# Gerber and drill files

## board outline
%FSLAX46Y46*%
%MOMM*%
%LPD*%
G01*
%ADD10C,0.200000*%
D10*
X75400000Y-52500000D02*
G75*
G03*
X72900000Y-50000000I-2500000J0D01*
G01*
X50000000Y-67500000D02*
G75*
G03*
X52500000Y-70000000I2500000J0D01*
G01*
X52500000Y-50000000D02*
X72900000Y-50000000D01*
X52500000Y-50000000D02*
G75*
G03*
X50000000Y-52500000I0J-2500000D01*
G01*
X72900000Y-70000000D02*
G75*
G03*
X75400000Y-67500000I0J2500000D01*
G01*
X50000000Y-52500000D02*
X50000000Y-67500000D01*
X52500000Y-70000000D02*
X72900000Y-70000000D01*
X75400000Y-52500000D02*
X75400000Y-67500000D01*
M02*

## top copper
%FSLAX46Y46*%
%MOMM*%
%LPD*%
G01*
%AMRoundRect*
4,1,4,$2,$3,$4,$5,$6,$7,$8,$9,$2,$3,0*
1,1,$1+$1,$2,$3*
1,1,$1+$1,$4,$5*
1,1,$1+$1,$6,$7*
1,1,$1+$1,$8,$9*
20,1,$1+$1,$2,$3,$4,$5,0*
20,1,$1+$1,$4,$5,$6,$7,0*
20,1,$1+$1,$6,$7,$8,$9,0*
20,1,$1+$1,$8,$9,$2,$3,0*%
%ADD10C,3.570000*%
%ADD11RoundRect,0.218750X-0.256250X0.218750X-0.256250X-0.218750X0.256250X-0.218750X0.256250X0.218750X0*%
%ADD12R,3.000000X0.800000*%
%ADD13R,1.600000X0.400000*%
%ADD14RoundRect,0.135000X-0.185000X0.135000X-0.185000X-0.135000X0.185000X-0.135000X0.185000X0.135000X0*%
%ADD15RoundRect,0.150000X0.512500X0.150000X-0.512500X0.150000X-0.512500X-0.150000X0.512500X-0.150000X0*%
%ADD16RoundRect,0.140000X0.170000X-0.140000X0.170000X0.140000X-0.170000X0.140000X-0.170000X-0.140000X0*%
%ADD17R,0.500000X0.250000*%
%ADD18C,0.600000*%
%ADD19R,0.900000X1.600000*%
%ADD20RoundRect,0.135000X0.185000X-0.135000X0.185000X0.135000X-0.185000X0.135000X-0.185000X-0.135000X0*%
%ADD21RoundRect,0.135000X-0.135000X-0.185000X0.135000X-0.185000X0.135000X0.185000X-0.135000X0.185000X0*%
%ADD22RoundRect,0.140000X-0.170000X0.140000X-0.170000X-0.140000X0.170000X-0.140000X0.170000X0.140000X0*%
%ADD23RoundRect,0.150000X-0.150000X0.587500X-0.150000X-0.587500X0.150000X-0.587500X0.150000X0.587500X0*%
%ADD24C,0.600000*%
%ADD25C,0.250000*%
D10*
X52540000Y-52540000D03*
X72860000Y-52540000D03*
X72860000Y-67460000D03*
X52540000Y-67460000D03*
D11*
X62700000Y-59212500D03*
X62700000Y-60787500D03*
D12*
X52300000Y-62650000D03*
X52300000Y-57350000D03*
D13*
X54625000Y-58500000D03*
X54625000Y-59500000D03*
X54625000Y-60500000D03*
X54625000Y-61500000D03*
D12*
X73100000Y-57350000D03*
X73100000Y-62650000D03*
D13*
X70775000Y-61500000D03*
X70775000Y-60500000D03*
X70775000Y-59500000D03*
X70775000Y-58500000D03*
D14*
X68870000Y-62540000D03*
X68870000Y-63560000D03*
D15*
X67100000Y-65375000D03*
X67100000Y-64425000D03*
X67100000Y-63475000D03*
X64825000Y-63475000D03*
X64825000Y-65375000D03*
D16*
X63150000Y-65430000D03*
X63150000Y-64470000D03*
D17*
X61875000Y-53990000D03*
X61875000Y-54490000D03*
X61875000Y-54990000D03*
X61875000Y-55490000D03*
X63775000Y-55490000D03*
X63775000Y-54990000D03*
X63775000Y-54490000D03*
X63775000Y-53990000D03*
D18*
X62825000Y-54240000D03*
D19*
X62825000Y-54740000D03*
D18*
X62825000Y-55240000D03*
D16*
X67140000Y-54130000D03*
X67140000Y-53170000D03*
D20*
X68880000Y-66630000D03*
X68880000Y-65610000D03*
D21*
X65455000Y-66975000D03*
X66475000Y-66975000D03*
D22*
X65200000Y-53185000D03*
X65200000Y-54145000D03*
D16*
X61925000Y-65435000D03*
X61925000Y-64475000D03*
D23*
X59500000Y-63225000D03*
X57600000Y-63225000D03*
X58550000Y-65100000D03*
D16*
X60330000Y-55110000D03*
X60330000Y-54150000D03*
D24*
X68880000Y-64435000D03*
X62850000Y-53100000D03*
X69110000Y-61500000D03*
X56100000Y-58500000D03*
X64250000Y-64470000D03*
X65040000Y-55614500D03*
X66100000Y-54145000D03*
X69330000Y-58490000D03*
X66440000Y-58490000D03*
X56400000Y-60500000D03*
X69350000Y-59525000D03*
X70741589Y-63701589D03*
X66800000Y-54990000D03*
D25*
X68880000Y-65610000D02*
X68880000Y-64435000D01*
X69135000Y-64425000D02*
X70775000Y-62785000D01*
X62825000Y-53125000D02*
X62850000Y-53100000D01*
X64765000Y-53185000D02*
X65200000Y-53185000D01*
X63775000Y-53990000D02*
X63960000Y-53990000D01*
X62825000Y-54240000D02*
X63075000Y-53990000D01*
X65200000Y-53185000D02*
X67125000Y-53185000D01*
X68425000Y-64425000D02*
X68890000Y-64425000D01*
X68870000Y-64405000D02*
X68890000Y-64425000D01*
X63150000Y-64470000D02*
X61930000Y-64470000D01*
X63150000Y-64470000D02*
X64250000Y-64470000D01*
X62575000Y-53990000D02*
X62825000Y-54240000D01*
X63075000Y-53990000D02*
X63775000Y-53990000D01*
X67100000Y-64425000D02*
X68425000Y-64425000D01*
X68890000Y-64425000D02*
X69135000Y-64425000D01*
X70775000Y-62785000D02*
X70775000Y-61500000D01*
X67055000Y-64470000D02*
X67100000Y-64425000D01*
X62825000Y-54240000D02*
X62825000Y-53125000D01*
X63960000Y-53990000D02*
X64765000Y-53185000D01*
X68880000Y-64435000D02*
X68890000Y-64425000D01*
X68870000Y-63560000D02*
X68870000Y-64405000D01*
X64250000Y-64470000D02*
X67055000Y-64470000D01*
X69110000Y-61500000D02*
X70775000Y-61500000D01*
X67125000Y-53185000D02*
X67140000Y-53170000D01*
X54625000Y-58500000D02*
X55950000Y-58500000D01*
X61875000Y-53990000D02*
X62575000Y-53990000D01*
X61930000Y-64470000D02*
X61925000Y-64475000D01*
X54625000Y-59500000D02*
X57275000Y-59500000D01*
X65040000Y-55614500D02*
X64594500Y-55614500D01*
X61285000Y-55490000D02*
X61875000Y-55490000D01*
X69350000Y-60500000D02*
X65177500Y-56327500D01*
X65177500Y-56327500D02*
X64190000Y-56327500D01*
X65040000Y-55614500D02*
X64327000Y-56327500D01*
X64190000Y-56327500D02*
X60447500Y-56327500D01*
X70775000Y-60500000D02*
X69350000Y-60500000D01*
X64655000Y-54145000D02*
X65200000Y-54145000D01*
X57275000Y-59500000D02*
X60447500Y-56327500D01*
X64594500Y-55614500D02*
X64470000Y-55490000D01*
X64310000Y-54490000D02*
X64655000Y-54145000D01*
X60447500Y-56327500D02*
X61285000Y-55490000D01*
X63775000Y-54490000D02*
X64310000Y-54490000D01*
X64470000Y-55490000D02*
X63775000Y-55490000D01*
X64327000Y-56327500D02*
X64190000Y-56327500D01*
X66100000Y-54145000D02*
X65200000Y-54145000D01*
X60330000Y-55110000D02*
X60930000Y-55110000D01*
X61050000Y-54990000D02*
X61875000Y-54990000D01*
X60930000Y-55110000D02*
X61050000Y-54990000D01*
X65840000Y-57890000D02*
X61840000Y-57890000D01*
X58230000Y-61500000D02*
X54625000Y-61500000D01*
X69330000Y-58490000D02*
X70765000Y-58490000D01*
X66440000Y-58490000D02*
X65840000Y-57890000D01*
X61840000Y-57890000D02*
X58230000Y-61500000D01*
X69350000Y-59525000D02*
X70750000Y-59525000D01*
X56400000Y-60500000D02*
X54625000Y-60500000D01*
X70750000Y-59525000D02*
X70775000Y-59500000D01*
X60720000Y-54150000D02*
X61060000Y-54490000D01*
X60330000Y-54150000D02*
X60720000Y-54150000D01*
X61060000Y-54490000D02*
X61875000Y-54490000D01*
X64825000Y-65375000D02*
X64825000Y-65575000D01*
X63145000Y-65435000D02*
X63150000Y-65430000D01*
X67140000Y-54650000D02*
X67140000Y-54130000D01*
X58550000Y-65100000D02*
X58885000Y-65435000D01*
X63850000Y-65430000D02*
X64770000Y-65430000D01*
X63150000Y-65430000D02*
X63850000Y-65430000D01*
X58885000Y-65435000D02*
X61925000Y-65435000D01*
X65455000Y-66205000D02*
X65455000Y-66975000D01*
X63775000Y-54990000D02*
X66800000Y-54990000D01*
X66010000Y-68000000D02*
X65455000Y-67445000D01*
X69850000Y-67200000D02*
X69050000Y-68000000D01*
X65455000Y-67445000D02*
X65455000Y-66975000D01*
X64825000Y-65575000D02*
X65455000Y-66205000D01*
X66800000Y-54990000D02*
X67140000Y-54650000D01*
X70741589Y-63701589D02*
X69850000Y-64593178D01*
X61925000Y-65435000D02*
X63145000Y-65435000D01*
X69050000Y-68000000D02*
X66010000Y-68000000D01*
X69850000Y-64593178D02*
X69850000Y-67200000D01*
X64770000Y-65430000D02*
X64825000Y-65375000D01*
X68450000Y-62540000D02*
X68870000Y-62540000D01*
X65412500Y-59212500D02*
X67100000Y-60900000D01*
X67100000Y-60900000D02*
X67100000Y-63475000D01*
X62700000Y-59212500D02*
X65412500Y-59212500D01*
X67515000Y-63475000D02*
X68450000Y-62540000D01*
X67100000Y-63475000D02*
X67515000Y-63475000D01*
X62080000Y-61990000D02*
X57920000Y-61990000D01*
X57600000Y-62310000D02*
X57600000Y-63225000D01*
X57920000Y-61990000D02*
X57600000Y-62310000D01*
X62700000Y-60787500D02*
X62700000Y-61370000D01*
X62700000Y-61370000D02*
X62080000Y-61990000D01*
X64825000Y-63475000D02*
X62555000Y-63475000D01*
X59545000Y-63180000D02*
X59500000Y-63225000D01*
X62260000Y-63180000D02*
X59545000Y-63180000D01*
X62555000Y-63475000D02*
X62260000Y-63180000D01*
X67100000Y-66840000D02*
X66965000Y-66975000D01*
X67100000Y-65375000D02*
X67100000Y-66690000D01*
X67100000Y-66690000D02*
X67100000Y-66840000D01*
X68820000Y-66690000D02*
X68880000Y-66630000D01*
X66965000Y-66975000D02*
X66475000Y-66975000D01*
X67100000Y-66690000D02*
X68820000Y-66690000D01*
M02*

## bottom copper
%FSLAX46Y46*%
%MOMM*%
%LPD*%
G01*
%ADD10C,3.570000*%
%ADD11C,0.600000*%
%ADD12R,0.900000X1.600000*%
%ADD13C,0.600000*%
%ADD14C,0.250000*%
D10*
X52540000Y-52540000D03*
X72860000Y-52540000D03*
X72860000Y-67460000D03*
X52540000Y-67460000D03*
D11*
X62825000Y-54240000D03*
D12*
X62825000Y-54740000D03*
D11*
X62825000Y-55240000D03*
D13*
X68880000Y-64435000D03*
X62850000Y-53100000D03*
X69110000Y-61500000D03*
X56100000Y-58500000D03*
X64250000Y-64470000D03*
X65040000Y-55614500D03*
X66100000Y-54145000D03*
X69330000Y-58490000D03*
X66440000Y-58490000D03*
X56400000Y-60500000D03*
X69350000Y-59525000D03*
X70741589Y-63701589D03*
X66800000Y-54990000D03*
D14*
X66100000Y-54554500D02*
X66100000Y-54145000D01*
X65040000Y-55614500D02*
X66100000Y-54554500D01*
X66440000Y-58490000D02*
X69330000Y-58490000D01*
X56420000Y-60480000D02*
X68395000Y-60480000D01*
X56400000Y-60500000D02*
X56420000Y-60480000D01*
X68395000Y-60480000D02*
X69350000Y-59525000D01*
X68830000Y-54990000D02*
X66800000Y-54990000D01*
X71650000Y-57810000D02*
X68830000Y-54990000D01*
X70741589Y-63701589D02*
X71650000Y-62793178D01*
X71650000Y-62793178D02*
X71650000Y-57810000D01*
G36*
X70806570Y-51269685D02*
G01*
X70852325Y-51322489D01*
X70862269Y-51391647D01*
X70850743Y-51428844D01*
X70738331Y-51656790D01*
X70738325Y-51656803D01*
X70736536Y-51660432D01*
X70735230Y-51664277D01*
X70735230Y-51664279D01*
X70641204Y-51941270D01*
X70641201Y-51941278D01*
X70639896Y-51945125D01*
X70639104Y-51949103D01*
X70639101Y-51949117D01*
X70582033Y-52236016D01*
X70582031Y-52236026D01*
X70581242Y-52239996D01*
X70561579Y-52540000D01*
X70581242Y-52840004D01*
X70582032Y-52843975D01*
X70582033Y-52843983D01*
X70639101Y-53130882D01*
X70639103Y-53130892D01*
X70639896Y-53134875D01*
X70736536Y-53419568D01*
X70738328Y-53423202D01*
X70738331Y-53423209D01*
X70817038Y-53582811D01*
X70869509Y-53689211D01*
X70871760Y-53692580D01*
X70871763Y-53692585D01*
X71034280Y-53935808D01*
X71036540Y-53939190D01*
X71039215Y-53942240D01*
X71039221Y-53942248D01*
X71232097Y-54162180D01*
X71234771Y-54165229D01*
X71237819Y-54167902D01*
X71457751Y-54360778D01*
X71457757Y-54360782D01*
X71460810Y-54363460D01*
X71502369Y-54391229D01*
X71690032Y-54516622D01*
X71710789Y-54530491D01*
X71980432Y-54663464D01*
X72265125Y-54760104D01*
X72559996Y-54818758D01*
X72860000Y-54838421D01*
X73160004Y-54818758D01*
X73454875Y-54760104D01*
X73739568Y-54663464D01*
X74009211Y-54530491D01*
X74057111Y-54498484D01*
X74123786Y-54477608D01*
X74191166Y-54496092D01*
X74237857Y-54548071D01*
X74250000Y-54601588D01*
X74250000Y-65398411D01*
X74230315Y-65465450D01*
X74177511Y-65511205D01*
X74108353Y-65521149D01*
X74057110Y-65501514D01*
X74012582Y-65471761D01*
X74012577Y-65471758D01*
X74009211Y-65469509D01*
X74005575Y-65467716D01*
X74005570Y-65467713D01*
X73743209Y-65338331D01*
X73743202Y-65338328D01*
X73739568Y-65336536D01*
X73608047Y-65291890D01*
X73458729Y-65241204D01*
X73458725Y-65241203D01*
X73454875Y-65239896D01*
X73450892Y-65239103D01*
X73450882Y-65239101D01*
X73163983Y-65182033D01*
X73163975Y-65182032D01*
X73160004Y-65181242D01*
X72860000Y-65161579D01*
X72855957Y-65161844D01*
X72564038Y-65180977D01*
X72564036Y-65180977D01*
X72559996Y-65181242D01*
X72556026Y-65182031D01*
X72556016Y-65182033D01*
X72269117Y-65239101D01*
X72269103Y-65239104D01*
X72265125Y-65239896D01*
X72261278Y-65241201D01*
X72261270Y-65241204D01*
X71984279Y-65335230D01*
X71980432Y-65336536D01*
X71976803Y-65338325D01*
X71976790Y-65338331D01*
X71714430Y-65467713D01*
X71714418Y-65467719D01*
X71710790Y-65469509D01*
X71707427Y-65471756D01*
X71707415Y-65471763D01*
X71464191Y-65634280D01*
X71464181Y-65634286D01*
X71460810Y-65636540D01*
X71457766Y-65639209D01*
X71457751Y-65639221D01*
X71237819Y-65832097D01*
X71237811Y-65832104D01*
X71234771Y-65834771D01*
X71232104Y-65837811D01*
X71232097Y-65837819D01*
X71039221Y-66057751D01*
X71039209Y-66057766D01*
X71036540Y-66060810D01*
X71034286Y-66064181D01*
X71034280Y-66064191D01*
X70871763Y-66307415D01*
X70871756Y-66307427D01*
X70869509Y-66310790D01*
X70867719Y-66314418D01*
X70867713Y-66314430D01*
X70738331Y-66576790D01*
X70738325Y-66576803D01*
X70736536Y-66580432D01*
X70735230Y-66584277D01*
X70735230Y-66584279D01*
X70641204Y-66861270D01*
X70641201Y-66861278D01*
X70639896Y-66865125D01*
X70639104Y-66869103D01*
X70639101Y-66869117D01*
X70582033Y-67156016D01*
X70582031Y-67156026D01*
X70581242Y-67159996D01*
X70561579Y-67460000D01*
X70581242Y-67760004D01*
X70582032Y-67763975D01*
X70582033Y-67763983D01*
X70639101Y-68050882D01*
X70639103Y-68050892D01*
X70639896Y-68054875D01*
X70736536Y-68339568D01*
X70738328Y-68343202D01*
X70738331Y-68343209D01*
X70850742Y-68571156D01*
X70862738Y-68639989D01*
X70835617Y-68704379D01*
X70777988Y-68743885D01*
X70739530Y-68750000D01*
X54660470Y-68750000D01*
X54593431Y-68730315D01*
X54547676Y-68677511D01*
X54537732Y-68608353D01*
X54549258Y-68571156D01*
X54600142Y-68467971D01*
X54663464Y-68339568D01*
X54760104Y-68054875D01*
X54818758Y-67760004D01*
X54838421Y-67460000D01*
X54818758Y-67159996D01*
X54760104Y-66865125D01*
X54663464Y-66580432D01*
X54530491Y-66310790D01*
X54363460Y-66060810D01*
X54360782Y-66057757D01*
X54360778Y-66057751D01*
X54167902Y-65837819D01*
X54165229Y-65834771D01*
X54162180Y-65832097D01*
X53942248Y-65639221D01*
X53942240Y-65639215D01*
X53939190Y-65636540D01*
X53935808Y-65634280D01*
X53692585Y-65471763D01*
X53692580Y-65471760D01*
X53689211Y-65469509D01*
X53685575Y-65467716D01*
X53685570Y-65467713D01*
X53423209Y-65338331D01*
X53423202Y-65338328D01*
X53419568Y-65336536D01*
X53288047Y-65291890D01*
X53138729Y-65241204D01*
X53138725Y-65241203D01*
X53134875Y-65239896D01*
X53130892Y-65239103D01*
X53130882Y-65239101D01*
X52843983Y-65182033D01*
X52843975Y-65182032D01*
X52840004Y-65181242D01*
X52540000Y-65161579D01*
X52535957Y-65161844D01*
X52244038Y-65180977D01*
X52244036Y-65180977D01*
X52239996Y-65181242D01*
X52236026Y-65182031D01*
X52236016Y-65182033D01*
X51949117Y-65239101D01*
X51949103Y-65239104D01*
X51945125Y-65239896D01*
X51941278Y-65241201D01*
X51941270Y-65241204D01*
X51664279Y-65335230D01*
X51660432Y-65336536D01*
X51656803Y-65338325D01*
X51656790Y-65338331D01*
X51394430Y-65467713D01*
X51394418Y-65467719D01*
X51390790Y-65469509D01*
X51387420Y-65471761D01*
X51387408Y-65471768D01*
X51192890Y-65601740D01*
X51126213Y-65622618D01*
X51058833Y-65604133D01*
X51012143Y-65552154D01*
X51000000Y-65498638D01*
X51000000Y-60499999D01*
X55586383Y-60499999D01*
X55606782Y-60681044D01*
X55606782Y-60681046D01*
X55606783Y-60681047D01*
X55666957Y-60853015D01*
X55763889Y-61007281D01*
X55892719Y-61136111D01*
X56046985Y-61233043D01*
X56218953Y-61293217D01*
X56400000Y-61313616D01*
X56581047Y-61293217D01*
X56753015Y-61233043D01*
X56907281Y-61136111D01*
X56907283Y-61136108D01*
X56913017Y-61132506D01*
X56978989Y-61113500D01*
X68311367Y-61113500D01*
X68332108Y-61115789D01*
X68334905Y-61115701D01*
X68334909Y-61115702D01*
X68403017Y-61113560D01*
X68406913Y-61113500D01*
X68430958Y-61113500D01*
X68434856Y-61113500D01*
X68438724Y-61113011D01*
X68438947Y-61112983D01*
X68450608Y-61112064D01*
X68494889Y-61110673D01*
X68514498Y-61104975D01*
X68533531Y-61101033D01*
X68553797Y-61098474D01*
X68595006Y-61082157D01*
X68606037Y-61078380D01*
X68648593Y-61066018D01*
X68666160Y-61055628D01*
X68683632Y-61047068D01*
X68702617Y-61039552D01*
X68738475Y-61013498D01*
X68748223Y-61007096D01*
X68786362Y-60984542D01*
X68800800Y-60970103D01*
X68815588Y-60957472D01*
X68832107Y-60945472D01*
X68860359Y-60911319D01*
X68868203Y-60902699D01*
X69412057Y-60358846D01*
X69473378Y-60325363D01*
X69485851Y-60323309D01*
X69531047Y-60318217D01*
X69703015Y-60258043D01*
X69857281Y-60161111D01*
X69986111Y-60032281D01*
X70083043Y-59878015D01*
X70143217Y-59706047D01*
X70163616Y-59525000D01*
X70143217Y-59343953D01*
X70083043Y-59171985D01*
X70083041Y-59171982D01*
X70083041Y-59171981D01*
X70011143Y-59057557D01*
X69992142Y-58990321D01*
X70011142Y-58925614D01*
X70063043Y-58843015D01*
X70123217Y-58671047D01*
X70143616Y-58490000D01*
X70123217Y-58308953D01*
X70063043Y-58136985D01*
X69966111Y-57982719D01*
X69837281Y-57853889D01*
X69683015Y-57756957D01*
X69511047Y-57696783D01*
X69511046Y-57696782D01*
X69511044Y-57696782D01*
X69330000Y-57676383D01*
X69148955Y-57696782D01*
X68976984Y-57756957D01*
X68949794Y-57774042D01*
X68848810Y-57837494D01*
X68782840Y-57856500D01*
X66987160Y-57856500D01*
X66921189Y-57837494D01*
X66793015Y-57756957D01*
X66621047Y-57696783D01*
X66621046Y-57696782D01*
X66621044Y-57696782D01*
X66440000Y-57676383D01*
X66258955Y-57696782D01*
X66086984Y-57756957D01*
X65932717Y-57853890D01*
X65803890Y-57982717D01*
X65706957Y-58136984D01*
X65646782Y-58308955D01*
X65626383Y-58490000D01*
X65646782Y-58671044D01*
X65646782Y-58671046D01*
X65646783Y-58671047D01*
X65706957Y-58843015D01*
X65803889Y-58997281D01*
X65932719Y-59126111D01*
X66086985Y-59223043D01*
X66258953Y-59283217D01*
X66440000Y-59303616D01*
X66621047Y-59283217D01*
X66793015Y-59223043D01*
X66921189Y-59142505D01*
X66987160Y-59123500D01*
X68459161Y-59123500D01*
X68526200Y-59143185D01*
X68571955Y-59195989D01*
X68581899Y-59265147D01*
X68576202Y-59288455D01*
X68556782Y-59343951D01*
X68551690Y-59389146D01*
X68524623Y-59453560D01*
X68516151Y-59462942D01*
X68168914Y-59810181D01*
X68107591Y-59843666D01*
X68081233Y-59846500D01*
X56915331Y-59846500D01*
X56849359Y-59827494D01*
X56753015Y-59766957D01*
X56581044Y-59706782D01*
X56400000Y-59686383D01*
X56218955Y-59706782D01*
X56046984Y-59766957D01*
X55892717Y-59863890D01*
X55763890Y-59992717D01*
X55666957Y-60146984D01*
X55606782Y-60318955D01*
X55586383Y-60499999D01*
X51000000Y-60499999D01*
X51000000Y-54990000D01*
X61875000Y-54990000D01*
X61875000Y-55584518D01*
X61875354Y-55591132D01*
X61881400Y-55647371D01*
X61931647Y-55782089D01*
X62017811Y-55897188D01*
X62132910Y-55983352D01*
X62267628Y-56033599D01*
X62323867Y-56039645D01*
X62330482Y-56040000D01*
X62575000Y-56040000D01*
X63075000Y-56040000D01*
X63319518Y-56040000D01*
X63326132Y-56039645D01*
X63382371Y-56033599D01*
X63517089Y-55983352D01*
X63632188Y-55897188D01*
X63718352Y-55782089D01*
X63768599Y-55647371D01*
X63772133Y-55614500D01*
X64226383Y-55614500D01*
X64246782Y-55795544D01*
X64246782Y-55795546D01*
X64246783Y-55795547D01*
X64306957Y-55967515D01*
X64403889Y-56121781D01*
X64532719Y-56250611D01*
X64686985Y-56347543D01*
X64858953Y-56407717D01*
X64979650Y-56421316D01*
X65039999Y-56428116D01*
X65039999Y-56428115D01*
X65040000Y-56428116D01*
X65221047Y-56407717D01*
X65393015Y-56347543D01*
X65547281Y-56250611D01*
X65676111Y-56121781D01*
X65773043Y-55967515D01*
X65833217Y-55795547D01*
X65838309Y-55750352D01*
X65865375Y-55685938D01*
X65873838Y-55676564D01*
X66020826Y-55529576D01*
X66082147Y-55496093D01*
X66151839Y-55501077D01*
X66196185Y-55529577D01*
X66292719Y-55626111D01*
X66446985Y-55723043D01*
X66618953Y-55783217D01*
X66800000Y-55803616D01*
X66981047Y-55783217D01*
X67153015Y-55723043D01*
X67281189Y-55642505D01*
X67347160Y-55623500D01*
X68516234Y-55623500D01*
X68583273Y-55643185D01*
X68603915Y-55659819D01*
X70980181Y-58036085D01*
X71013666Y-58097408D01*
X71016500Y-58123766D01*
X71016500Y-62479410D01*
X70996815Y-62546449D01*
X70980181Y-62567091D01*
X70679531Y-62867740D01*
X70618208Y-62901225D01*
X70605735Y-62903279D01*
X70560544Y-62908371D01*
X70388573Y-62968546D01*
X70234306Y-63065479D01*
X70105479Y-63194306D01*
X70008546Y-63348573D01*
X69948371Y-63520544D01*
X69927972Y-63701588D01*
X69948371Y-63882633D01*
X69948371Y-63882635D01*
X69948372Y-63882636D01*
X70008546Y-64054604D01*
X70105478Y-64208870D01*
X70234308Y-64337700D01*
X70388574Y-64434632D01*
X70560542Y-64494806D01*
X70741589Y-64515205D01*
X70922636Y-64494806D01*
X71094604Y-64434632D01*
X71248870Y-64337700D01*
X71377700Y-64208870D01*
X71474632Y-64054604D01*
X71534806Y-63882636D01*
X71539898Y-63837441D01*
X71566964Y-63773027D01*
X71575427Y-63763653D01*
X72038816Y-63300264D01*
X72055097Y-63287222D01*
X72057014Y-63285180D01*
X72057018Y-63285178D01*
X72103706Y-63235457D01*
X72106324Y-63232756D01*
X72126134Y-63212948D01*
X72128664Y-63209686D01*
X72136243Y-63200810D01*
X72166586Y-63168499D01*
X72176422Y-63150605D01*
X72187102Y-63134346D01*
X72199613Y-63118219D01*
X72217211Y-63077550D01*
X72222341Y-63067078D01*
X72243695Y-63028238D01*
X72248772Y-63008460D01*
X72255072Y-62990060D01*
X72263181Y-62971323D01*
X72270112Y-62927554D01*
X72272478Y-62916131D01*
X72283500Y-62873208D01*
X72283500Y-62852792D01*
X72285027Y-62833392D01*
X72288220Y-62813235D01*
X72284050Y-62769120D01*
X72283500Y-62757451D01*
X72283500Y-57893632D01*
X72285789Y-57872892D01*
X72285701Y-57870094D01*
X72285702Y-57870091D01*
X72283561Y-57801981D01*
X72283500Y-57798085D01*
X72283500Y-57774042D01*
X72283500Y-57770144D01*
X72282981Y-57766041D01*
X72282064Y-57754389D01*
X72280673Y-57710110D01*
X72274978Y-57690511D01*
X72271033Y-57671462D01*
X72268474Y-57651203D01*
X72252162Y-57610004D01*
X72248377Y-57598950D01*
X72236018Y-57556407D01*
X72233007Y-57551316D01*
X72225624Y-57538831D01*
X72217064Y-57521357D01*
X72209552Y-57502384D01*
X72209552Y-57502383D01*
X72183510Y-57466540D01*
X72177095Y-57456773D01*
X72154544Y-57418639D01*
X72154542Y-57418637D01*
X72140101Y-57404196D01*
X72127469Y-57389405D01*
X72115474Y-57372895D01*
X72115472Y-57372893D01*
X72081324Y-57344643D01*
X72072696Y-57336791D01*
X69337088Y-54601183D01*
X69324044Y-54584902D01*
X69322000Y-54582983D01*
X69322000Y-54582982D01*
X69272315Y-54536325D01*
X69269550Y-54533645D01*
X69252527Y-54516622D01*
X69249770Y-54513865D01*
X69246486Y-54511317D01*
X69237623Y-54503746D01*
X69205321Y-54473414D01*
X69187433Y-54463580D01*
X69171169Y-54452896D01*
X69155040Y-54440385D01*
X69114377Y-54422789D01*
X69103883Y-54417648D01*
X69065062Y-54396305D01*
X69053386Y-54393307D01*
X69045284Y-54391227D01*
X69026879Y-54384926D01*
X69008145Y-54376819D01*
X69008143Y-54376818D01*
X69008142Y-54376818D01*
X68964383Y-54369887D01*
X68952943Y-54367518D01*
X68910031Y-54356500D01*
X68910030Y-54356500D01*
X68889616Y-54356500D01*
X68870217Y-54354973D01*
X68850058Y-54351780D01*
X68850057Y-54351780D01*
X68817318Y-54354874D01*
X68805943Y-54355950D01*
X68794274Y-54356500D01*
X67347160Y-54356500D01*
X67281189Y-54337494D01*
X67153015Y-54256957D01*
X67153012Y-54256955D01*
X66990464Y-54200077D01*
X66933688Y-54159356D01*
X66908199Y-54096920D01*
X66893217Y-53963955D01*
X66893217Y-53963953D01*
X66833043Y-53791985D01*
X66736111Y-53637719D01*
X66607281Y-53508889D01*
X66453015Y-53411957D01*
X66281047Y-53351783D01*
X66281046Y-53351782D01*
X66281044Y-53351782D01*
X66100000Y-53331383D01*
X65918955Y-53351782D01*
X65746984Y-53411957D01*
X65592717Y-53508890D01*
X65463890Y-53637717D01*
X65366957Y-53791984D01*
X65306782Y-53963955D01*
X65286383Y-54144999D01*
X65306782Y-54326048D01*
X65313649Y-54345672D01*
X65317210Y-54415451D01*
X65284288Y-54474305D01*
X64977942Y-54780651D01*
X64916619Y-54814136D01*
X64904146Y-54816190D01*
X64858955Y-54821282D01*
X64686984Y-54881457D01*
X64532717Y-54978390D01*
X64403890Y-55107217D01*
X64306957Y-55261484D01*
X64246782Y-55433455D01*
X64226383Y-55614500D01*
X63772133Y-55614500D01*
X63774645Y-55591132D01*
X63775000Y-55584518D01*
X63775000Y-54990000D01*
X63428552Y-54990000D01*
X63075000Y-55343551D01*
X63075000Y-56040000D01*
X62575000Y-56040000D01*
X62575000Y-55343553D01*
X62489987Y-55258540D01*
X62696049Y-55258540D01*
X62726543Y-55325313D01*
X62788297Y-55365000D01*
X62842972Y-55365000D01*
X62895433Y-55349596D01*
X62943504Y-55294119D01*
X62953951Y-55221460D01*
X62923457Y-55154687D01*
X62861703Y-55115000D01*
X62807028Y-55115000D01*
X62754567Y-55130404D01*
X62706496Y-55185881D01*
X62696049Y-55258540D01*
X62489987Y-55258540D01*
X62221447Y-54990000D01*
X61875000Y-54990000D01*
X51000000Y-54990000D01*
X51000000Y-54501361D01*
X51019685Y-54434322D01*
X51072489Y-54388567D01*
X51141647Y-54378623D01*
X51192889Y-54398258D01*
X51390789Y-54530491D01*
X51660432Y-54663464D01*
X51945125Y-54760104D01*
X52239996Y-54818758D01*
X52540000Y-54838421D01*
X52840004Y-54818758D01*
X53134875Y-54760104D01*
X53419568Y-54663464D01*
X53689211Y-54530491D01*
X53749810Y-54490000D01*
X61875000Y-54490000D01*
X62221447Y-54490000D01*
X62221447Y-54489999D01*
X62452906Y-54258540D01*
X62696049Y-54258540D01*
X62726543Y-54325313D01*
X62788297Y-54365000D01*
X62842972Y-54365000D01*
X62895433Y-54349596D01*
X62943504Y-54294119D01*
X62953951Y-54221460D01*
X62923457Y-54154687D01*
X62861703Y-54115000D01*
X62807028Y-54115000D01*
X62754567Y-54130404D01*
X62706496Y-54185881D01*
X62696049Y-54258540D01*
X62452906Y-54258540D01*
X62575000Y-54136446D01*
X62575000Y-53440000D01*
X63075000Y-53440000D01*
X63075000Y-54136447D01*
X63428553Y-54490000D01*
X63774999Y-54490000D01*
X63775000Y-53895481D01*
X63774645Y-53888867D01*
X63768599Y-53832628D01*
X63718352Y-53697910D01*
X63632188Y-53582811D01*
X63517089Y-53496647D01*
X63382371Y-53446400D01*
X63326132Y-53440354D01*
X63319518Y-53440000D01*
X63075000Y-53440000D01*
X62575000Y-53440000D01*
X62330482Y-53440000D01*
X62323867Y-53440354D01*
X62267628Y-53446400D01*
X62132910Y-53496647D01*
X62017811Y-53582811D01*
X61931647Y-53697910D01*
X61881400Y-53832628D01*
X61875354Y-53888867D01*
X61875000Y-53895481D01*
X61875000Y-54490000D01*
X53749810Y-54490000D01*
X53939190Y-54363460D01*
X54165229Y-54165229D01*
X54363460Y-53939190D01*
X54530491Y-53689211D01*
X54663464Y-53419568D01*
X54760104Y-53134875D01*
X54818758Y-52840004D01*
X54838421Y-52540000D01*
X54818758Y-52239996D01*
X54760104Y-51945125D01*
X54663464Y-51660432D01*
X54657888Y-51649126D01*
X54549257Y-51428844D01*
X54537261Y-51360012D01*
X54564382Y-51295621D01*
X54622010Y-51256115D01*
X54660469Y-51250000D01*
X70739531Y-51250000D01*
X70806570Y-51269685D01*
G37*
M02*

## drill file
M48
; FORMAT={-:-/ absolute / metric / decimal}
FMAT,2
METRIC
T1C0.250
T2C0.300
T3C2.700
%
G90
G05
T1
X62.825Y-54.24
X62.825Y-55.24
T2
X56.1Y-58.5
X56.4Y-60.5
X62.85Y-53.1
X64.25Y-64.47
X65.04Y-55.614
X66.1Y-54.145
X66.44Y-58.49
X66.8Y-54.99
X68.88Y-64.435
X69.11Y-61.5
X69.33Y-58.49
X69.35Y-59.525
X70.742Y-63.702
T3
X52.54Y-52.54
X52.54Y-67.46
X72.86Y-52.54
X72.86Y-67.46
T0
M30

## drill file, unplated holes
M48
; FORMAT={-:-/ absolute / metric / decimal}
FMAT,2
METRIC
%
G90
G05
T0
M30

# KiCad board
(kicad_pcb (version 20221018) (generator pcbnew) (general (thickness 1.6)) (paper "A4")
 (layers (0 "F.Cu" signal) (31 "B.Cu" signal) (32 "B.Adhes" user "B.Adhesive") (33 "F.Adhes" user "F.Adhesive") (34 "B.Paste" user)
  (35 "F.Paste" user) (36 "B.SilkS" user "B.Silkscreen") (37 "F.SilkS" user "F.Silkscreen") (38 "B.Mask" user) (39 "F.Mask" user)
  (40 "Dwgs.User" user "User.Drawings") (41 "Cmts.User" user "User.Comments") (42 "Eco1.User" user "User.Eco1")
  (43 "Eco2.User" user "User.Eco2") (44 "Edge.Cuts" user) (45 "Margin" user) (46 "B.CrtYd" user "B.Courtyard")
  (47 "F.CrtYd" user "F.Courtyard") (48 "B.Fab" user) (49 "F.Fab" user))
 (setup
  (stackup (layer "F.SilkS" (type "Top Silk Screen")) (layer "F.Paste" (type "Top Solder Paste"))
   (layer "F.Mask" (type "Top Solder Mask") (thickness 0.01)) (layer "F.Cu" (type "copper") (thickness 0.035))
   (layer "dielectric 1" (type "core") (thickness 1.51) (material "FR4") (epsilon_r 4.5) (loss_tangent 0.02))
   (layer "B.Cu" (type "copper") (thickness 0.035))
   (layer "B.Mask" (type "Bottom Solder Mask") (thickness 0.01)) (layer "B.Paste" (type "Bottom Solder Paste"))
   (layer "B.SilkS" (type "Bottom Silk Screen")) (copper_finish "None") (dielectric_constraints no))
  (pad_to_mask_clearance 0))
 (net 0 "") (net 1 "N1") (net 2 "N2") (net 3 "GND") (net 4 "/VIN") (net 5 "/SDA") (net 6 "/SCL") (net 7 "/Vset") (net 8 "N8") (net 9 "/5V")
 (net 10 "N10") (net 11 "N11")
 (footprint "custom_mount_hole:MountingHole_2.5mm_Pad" (layer "F.Cu") (at 52.54 52.54)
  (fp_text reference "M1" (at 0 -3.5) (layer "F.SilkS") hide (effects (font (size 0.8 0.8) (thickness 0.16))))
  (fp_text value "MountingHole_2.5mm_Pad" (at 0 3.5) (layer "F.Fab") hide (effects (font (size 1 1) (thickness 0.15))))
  (pad "~" thru_hole circle (at 0 0) (size 3.57 3.57) (drill 2.7) (layers "*.Cu" "*.Mask")))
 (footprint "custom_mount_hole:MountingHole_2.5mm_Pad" (layer "F.Cu") (at 72.86 52.54)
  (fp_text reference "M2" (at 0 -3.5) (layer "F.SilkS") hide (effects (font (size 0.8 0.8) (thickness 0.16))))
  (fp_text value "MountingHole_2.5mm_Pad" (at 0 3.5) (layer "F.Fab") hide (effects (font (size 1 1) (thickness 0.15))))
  (pad "~" thru_hole circle (at 0 0) (size 3.57 3.57) (drill 2.7) (layers "*.Cu" "*.Mask")))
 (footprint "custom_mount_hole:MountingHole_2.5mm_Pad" (layer "F.Cu") (at 72.86 67.46)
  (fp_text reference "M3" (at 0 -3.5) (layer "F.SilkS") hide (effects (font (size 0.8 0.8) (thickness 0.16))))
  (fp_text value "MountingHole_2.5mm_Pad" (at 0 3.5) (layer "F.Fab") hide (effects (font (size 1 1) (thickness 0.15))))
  (pad "~" thru_hole circle (at 0 0) (size 3.57 3.57) (drill 2.7) (layers "*.Cu" "*.Mask")))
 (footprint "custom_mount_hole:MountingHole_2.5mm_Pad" (layer "F.Cu") (at 52.54 67.46)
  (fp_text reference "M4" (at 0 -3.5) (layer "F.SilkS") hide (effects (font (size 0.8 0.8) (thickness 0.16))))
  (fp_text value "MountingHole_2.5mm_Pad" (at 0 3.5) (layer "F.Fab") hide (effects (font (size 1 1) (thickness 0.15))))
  (pad "~" thru_hole circle (at 0 0) (size 3.57 3.57) (drill 2.7) (layers "*.Cu" "*.Mask")))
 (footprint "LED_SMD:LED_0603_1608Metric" (layer "F.Cu") (at 62.7 60 -90)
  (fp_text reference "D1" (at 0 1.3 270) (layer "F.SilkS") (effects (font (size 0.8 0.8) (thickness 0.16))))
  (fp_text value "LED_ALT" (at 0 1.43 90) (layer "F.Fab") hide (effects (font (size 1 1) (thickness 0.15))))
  (pad "1" smd roundrect (at -0.7875 0 270) (size 0.875 0.95) (layers "F.Cu" "F.Paste" "F.Mask") (roundrect_rratio 0.25) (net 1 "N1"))
  (pad "2" smd roundrect (at 0.7875 0 270) (size 0.875 0.95) (layers "F.Cu" "F.Paste" "F.Mask") (roundrect_rratio 0.25) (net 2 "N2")))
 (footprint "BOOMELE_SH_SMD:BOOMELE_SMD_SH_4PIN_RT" (layer "F.Cu") (at 52.78 60 90)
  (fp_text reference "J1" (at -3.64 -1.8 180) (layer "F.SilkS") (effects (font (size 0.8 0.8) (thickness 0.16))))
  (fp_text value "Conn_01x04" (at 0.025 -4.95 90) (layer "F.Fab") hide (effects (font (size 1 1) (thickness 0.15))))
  (pad "" smd rect (at -2.65 -0.48 270) (size 0.8 3) (layers "F.Cu" "F.Paste" "F.Mask"))
  (pad "" smd rect (at 2.65 -0.48 270) (size 0.8 3) (layers "F.Cu" "F.Paste" "F.Mask"))
  (pad "1" smd rect (at 1.5 1.845 270) (size 0.4 1.6) (layers "F.Cu" "F.Paste" "F.Mask") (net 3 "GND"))
  (pad "2" smd rect (at 0.5 1.845 270) (size 0.4 1.6) (layers "F.Cu" "F.Paste" "F.Mask") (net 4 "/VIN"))
  (pad "3" smd rect (at -0.5 1.845 270) (size 0.4 1.6) (layers "F.Cu" "F.Paste" "F.Mask") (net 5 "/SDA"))
  (pad "4" smd rect (at -1.5 1.845 270) (size 0.4 1.6) (layers "F.Cu" "F.Paste" "F.Mask") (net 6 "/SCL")))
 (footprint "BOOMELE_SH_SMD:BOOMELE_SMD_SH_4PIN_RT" (layer "F.Cu") (at 72.62 60 -90)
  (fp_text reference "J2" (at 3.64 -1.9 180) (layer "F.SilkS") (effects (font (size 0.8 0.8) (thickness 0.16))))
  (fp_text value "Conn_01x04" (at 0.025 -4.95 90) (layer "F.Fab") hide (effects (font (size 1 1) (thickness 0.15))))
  (pad "" smd rect (at -2.65 -0.48 90) (size 0.8 3) (layers "F.Cu" "F.Paste" "F.Mask"))
  (pad "" smd rect (at 2.65 -0.48 90) (size 0.8 3) (layers "F.Cu" "F.Paste" "F.Mask"))
  (pad "1" smd rect (at 1.5 1.845 90) (size 0.4 1.6) (layers "F.Cu" "F.Paste" "F.Mask") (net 3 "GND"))
  (pad "2" smd rect (at 0.5 1.845 90) (size 0.4 1.6) (layers "F.Cu" "F.Paste" "F.Mask") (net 4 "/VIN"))
  (pad "3" smd rect (at -0.5 1.845 90) (size 0.4 1.6) (layers "F.Cu" "F.Paste" "F.Mask") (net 5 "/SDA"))
  (pad "4" smd rect (at -1.5 1.845 90) (size 0.4 1.6) (layers "F.Cu" "F.Paste" "F.Mask") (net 6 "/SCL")))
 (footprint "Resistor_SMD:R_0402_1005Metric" (layer "F.Cu") (at 68.87 63.05 -90)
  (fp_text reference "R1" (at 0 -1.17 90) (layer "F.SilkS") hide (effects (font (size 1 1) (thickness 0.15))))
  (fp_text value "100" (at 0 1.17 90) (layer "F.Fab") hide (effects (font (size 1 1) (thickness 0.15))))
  (pad "1" smd roundrect (at -0.51 0 270) (size 0.54 0.64) (layers "F.Cu" "F.Paste" "F.Mask") (roundrect_rratio 0.25) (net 1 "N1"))
  (pad "2" smd roundrect (at 0.51 0 270) (size 0.54 0.64) (layers "F.Cu" "F.Paste" "F.Mask") (roundrect_rratio 0.25) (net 3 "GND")))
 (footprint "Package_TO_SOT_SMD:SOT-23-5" (layer "F.Cu") (at 65.9625 64.425 180)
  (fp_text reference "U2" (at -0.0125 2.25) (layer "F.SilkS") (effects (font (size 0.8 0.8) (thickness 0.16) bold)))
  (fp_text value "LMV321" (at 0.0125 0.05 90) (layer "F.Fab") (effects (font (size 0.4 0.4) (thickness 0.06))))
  (pad "1" smd roundrect (at -1.1375 -0.95 180) (size 1.325 0.6) (layers "F.Cu" "F.Paste" "F.Mask") (roundrect_rratio 0.25) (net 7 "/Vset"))
  (pad "2" smd roundrect (at -1.1375 0 180) (size 1.325 0.6) (layers "F.Cu" "F.Paste" "F.Mask") (roundrect_rratio 0.25) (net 3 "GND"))
  (pad "3" smd roundrect (at -1.1375 0.95 180) (size 1.325 0.6) (layers "F.Cu" "F.Paste" "F.Mask") (roundrect_rratio 0.25) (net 1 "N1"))
  (pad "4" smd roundrect (at 1.1375 0.95 180) (size 1.325 0.6) (layers "F.Cu" "F.Paste" "F.Mask") (roundrect_rratio 0.25) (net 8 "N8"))
  (pad "5" smd roundrect (at 1.1375 -0.95 180) (size 1.325 0.6) (layers "F.Cu" "F.Paste" "F.Mask") (roundrect_rratio 0.25) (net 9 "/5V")))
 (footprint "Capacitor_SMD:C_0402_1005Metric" (layer "F.Cu") (at 63.15 64.95 90)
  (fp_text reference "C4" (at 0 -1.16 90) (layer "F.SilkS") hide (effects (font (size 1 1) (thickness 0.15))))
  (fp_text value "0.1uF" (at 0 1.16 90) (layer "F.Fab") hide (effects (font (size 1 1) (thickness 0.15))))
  (pad "1" smd roundrect (at -0.48 0 90) (size 0.56 0.62) (layers "F.Cu" "F.Paste" "F.Mask") (roundrect_rratio 0.25) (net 9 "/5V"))
  (pad "2" smd roundrect (at 0.48 0 90) (size 0.56 0.62) (layers "F.Cu" "F.Paste" "F.Mask") (roundrect_rratio 0.25) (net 3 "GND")))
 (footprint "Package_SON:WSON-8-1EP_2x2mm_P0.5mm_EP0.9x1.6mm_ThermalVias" (layer "F.Cu") (at 62.825 54.74)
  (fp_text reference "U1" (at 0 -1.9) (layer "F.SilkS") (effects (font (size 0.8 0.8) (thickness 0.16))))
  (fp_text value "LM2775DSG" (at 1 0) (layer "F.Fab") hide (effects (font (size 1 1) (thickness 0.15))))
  (pad "" smd rect (at 0 -0.4) (size 0.75 0.65) (layers "F.Paste"))
  (pad "" smd rect (at 0 0.4) (size 0.75 0.65) (layers "F.Paste"))
  (pad "1" smd rect (at -0.95 -0.75) (size 0.5 0.25) (layers "F.Cu" "F.Paste" "F.Mask") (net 3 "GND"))
  (pad "2" smd rect (at -0.95 -0.25) (size 0.5 0.25) (layers "F.Cu" "F.Paste" "F.Mask") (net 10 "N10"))
  (pad "3" smd rect (at -0.95 0.25) (size 0.5 0.25) (layers "F.Cu" "F.Paste" "F.Mask") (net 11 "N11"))
  (pad "4" smd rect (at -0.95 0.75) (size 0.5 0.25) (layers "F.Cu" "F.Paste" "F.Mask") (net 4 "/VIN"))
  (pad "5" smd rect (at 0.95 0.75) (size 0.5 0.25) (layers "F.Cu" "F.Paste" "F.Mask") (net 4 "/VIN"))
  (pad "6" smd rect (at 0.95 0.25) (size 0.5 0.25) (layers "F.Cu" "F.Paste" "F.Mask") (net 9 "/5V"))
  (pad "7" smd rect (at 0.95 -0.25) (size 0.5 0.25) (layers "F.Cu" "F.Paste" "F.Mask") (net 4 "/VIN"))
  (pad "8" smd rect (at 0.95 -0.75) (size 0.5 0.25) (layers "F.Cu" "F.Paste" "F.Mask") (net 3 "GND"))
  (pad "9" thru_hole circle (at 0 -0.5) (size 0.6 0.6) (drill 0.25) (layers "*.Cu") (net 3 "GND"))
  (pad "9" smd rect (at 0 0) (size 0.9 1.6) (layers "F.Cu" "F.Mask") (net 3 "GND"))
  (pad "9" smd rect (at 0 0) (size 0.9 1.6) (layers "B.Cu") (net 3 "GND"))
  (pad "9" thru_hole circle (at 0 0.5) (size 0.6 0.6) (drill 0.25) (layers "*.Cu") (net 3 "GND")))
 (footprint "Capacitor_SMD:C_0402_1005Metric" (layer "F.Cu") (at 67.14 53.65 90)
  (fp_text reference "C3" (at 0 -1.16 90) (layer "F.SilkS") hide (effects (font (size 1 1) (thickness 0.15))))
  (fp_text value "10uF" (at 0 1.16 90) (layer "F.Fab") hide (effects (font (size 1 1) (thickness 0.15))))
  (pad "1" smd roundrect (at -0.48 0 90) (size 0.56 0.62) (layers "F.Cu" "F.Paste" "F.Mask") (roundrect_rratio 0.25) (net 9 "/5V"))
  (pad "2" smd roundrect (at 0.48 0 90) (size 0.56 0.62) (layers "F.Cu" "F.Paste" "F.Mask") (roundrect_rratio 0.25) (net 3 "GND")))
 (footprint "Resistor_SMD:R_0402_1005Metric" (layer "F.Cu") (at 68.88 66.12 90)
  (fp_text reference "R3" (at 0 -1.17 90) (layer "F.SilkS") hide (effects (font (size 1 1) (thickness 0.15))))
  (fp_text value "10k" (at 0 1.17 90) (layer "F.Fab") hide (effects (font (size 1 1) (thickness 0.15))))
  (pad "1" smd roundrect (at -0.51 0 90) (size 0.54 0.64) (layers "F.Cu" "F.Paste" "F.Mask") (roundrect_rratio 0.25) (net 7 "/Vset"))
  (pad "2" smd roundrect (at 0.51 0 90) (size 0.54 0.64) (layers "F.Cu" "F.Paste" "F.Mask") (roundrect_rratio 0.25) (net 3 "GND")))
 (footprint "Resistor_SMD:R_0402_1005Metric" (layer "F.Cu") (at 65.965 66.975)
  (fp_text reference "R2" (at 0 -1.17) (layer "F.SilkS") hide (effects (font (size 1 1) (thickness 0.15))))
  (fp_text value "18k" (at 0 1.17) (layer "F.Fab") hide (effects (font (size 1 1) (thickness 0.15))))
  (pad "1" smd roundrect (at -0.51 0) (size 0.54 0.64) (layers "F.Cu" "F.Paste" "F.Mask") (roundrect_rratio 0.25) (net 9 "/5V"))
  (pad "2" smd roundrect (at 0.51 0) (size 0.54 0.64) (layers "F.Cu" "F.Paste" "F.Mask") (roundrect_rratio 0.25) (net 7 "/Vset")))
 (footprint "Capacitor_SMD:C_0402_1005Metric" (layer "F.Cu") (at 65.2 53.665 -90)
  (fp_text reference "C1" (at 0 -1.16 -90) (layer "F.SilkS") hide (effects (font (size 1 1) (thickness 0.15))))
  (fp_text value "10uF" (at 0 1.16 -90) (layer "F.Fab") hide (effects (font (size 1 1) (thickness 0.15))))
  (pad "1" smd roundrect (at -0.48 0 270) (size 0.56 0.62) (layers "F.Cu" "F.Paste" "F.Mask") (roundrect_rratio 0.25) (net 3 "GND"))
  (pad "2" smd roundrect (at 0.48 0 270) (size 0.56 0.62) (layers "F.Cu" "F.Paste" "F.Mask") (roundrect_rratio 0.25) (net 4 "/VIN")))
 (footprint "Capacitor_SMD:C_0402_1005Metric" (layer "F.Cu") (at 61.925 64.955 90)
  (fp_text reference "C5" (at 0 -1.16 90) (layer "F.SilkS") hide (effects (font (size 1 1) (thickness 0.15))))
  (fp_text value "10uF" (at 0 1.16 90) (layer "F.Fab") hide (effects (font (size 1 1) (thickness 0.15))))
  (pad "1" smd roundrect (at -0.48 0 90) (size 0.56 0.62) (layers "F.Cu" "F.Paste" "F.Mask") (roundrect_rratio 0.25) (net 9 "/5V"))
  (pad "2" smd roundrect (at 0.48 0 90) (size 0.56 0.62) (layers "F.Cu" "F.Paste" "F.Mask") (roundrect_rratio 0.25) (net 3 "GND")))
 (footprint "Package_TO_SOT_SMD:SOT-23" (layer "F.Cu") (at 58.55 64.1625 -90)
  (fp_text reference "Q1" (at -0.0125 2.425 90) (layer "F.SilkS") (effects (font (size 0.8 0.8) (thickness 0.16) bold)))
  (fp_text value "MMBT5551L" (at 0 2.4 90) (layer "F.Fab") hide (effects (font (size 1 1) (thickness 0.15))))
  (pad "1" smd roundrect (at -0.9375 -0.95 270) (size 1.475 0.6) (layers "F.Cu" "F.Paste" "F.Mask") (roundrect_rratio 0.25) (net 8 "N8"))
  (pad "2" smd roundrect (at -0.9375 0.95 270) (size 1.475 0.6) (layers "F.Cu" "F.Paste" "F.Mask") (roundrect_rratio 0.25) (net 2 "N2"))
  (pad "3" smd roundrect (at 0.9375 0 270) (size 1.475 0.6) (layers "F.Cu" "F.Paste" "F.Mask") (roundrect_rratio 0.25) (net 9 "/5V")))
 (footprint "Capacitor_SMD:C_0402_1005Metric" (layer "F.Cu") (at 60.33 54.63 90)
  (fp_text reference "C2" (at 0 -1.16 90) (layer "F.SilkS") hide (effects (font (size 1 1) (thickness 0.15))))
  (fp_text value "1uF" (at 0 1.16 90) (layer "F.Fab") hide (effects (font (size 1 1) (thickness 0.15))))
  (pad "1" smd roundrect (at -0.48 0 90) (size 0.56 0.62) (layers "F.Cu" "F.Paste" "F.Mask") (roundrect_rratio 0.25) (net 11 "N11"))
  (pad "2" smd roundrect (at 0.48 0 90) (size 0.56 0.62) (layers "F.Cu" "F.Paste" "F.Mask") (roundrect_rratio 0.25) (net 10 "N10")))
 (gr_arc (start 72.9 50) (mid 74.667767 50.732233) (end 75.4 52.5) (stroke (width 0.2) (type solid)) (layer "Edge.Cuts"))
 (gr_arc (start 52.5 70) (mid 50.732233 69.267767) (end 50 67.5) (stroke (width 0.2) (type solid)) (layer "Edge.Cuts"))
 (gr_line (start 52.5 50) (end 72.9 50) (stroke (width 0.2) (type solid)) (layer "Edge.Cuts"))
 (gr_arc (start 50 52.5) (mid 50.732233 50.732233) (end 52.5 50) (stroke (width 0.2) (type solid)) (layer "Edge.Cuts"))
 (gr_arc (start 75.4 67.5) (mid 74.667767 69.267767) (end 72.9 70) (stroke (width 0.2) (type solid)) (layer "Edge.Cuts"))
 (gr_line (start 50 52.5) (end 50 67.5) (stroke (width 0.2) (type solid)) (layer "Edge.Cuts"))
 (gr_line (start 52.5 70) (end 72.9 70) (stroke (width 0.2) (type solid)) (layer "Edge.Cuts"))
 (gr_line (start 75.4 52.5) (end 75.4 67.5) (stroke (width 0.2) (type solid)) (layer "Edge.Cuts"))
 (segment (start 68.88 65.61) (end 68.88 64.435) (width 0.25) (layer "F.Cu") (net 3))
 (segment (start 69.135 64.425) (end 70.775 62.785) (width 0.25) (layer "F.Cu") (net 3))
 (segment (start 62.825 53.125) (end 62.85 53.1) (width 0.25) (layer "F.Cu") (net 3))
 (segment (start 64.765 53.185) (end 65.2 53.185) (width 0.25) (layer "F.Cu") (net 3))
 (segment (start 63.775 53.99) (end 63.96 53.99) (width 0.25) (layer "F.Cu") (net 3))
 (segment (start 62.825 54.24) (end 63.075 53.99) (width 0.25) (layer "F.Cu") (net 3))
 (segment (start 65.2 53.185) (end 67.125 53.185) (width 0.25) (layer "F.Cu") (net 3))
 (segment (start 68.425 64.425) (end 68.89 64.425) (width 0.25) (layer "F.Cu") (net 3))
 (segment (start 68.87 64.405) (end 68.89 64.425) (width 0.25) (layer "F.Cu") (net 3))
 (segment (start 63.15 64.47) (end 61.93 64.47) (width 0.25) (layer "F.Cu") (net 3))
 (segment (start 63.15 64.47) (end 64.25 64.47) (width 0.25) (layer "F.Cu") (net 3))
 (segment (start 62.575 53.99) (end 62.825 54.24) (width 0.25) (layer "F.Cu") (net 3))
 (segment (start 63.075 53.99) (end 63.775 53.99) (width 0.25) (layer "F.Cu") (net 3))
 (segment (start 67.1 64.425) (end 68.425 64.425) (width 0.25) (layer "F.Cu") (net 3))
 (segment (start 68.89 64.425) (end 69.135 64.425) (width 0.25) (layer "F.Cu") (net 3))
 (segment (start 70.775 62.785) (end 70.775 61.5) (width 0.25) (layer "F.Cu") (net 3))
 (segment (start 67.055 64.47) (end 67.1 64.425) (width 0.25) (layer "F.Cu") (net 3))
 (segment (start 62.825 54.24) (end 62.825 53.125) (width 0.25) (layer "F.Cu") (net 3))
 (segment (start 63.96 53.99) (end 64.765 53.185) (width 0.25) (layer "F.Cu") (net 3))
 (segment (start 68.88 64.435) (end 68.89 64.425) (width 0.25) (layer "F.Cu") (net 3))
 (segment (start 68.87 63.56) (end 68.87 64.405) (width 0.25) (layer "F.Cu") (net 3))
 (segment (start 64.25 64.47) (end 67.055 64.47) (width 0.25) (layer "F.Cu") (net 3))
 (segment (start 69.11 61.5) (end 70.775 61.5) (width 0.25) (layer "F.Cu") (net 3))
 (segment (start 67.125 53.185) (end 67.14 53.17) (width 0.25) (layer "F.Cu") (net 3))
 (segment (start 54.625 58.5) (end 55.95 58.5) (width 0.25) (layer "F.Cu") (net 3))
 (segment (start 61.875 53.99) (end 62.575 53.99) (width 0.25) (layer "F.Cu") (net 3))
 (segment (start 61.93 64.47) (end 61.925 64.475) (width 0.25) (layer "F.Cu") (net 3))
 (via (at 68.88 64.435) (size 0.6) (drill 0.3) (layers "F.Cu" "B.Cu") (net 3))
 (via (at 62.85 53.1) (size 0.6) (drill 0.3) (layers "F.Cu" "B.Cu") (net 3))
 (via (at 69.11 61.5) (size 0.6) (drill 0.3) (layers "F.Cu" "B.Cu") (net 3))
 (via (at 56.1 58.5) (size 0.6) (drill 0.3) (layers "F.Cu" "B.Cu") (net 3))
 (via (at 64.25 64.47) (size 0.6) (drill 0.3) (layers "F.Cu" "B.Cu") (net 3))
 (segment (start 54.625 59.5) (end 57.275 59.5) (width 0.25) (layer "F.Cu") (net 4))
 (segment (start 65.04 55.6145) (end 64.5945 55.6145) (width 0.25) (layer "F.Cu") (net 4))
 (segment (start 61.285 55.49) (end 61.875 55.49) (width 0.25) (layer "F.Cu") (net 4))
 (segment (start 69.35 60.5) (end 65.1775 56.3275) (width 0.25) (layer "F.Cu") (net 4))
 (segment (start 65.1775 56.3275) (end 64.19 56.3275) (width 0.25) (layer "F.Cu") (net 4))
 (segment (start 65.04 55.6145) (end 64.327 56.3275) (width 0.25) (layer "F.Cu") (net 4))
 (segment (start 64.19 56.3275) (end 60.4475 56.3275) (width 0.25) (layer "F.Cu") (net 4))
 (segment (start 70.775 60.5) (end 69.35 60.5) (width 0.25) (layer "F.Cu") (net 4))
 (segment (start 64.655 54.145) (end 65.2 54.145) (width 0.25) (layer "F.Cu") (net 4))
 (segment (start 57.275 59.5) (end 60.4475 56.3275) (width 0.25) (layer "F.Cu") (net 4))
 (segment (start 64.5945 55.6145) (end 64.47 55.49) (width 0.25) (layer "F.Cu") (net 4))
 (segment (start 64.31 54.49) (end 64.655 54.145) (width 0.25) (layer "F.Cu") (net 4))
 (segment (start 60.4475 56.3275) (end 61.285 55.49) (width 0.25) (layer "F.Cu") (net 4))
 (segment (start 63.775 54.49) (end 64.31 54.49) (width 0.25) (layer "F.Cu") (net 4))
 (segment (start 64.47 55.49) (end 63.775 55.49) (width 0.25) (layer "F.Cu") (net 4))
 (segment (start 64.327 56.3275) (end 64.19 56.3275) (width 0.25) (layer "F.Cu") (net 4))
 (segment (start 66.1 54.145) (end 65.2 54.145) (width 0.25) (layer "F.Cu") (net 4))
 (via (at 65.04 55.6145) (size 0.6) (drill 0.3) (layers "F.Cu" "B.Cu") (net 4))
 (via (at 66.1 54.145) (size 0.6) (drill 0.3) (layers "F.Cu" "B.Cu") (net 4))
 (segment (start 66.1 54.5545) (end 66.1 54.145) (width 0.25) (layer "B.Cu") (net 4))
 (segment (start 65.04 55.6145) (end 66.1 54.5545) (width 0.25) (layer "B.Cu") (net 4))
 (segment (start 60.33 55.11) (end 60.93 55.11) (width 0.25) (layer "F.Cu") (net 11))
 (segment (start 61.05 54.99) (end 61.875 54.99) (width 0.25) (layer "F.Cu") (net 11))
 (segment (start 60.93 55.11) (end 61.05 54.99) (width 0.25) (layer "F.Cu") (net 11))
 (segment (start 65.84 57.89) (end 61.84 57.89) (width 0.25) (layer "F.Cu") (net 6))
 (segment (start 58.23 61.5) (end 54.625 61.5) (width 0.25) (layer "F.Cu") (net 6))
 (segment (start 69.33 58.49) (end 70.765 58.49) (width 0.25) (layer "F.Cu") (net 6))
 (segment (start 66.44 58.49) (end 65.84 57.89) (width 0.25) (layer "F.Cu") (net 6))
 (segment (start 61.84 57.89) (end 58.23 61.5) (width 0.25) (layer "F.Cu") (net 6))
 (via (at 69.33 58.49) (size 0.6) (drill 0.3) (layers "F.Cu" "B.Cu") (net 6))
 (via (at 66.44 58.49) (size 0.6) (drill 0.3) (layers "F.Cu" "B.Cu") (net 6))
 (segment (start 66.44 58.49) (end 69.33 58.49) (width 0.25) (layer "B.Cu") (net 6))
 (segment (start 69.35 59.525) (end 70.75 59.525) (width 0.25) (layer "F.Cu") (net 5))
 (segment (start 56.4 60.5) (end 54.625 60.5) (width 0.25) (layer "F.Cu") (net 5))
 (segment (start 70.75 59.525) (end 70.775 59.5) (width 0.25) (layer "F.Cu") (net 5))
 (via (at 56.4 60.5) (size 0.6) (drill 0.3) (layers "F.Cu" "B.Cu") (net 5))
 (via (at 69.35 59.525) (size 0.6) (drill 0.3) (layers "F.Cu" "B.Cu") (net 5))
 (segment (start 56.42 60.48) (end 68.395 60.48) (width 0.25) (layer "B.Cu") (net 5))
 (segment (start 56.4 60.5) (end 56.42 60.48) (width 0.25) (layer "B.Cu") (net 5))
 (segment (start 68.395 60.48) (end 69.35 59.525) (width 0.25) (layer "B.Cu") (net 5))
 (segment (start 60.72 54.15) (end 61.06 54.49) (width 0.25) (layer "F.Cu") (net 10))
 (segment (start 60.33 54.15) (end 60.72 54.15) (width 0.25) (layer "F.Cu") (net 10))
 (segment (start 61.06 54.49) (end 61.875 54.49) (width 0.25) (layer "F.Cu") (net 10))
 (segment (start 64.825 65.375) (end 64.825 65.575) (width 0.25) (layer "F.Cu") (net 9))
 (segment (start 63.145 65.435) (end 63.15 65.43) (width 0.25) (layer "F.Cu") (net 9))
 (segment (start 67.14 54.65) (end 67.14 54.13) (width 0.25) (layer "F.Cu") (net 9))
 (segment (start 58.55 65.1) (end 58.885 65.435) (width 0.25) (layer "F.Cu") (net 9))
 (segment (start 63.85 65.43) (end 64.77 65.43) (width 0.25) (layer "F.Cu") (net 9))
 (segment (start 63.15 65.43) (end 63.85 65.43) (width 0.25) (layer "F.Cu") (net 9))
 (segment (start 58.885 65.435) (end 61.925 65.435) (width 0.25) (layer "F.Cu") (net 9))
 (segment (start 65.455 66.205) (end 65.455 66.975) (width 0.25) (layer "F.Cu") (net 9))
 (segment (start 63.775 54.99) (end 66.8 54.99) (width 0.25) (layer "F.Cu") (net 9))
 (segment (start 66.01 68) (end 65.455 67.445) (width 0.25) (layer "F.Cu") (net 9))
 (segment (start 69.85 67.2) (end 69.05 68) (width 0.25) (layer "F.Cu") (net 9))
 (segment (start 65.455 67.445) (end 65.455 66.975) (width 0.25) (layer "F.Cu") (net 9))
 (segment (start 64.825 65.575) (end 65.455 66.205) (width 0.25) (layer "F.Cu") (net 9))
 (segment (start 66.8 54.99) (end 67.14 54.65) (width 0.25) (layer "F.Cu") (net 9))
 (segment (start 70.741589 63.701589) (end 69.85 64.593178) (width 0.25) (layer "F.Cu") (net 9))
 (segment (start 61.925 65.435) (end 63.145 65.435) (width 0.25) (layer "F.Cu") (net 9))
 (segment (start 69.05 68) (end 66.01 68) (width 0.25) (layer "F.Cu") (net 9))
 (segment (start 69.85 64.593178) (end 69.85 67.2) (width 0.25) (layer "F.Cu") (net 9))
 (segment (start 64.77 65.43) (end 64.825 65.375) (width 0.25) (layer "F.Cu") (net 9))
 (via (at 70.741589 63.701589) (size 0.6) (drill 0.3) (layers "F.Cu" "B.Cu") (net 9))
 (via (at 66.8 54.99) (size 0.6) (drill 0.3) (layers "F.Cu" "B.Cu") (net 9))
 (segment (start 68.83 54.99) (end 66.8 54.99) (width 0.25) (layer "B.Cu") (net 9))
 (segment (start 71.65 57.81) (end 68.83 54.99) (width 0.25) (layer "B.Cu") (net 9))
 (segment (start 70.741589 63.701589) (end 71.65 62.793178) (width 0.25) (layer "B.Cu") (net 9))
 (segment (start 71.65 62.793178) (end 71.65 57.81) (width 0.25) (layer "B.Cu") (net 9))
 (segment (start 68.45 62.54) (end 68.87 62.54) (width 0.25) (layer "F.Cu") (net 1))
 (segment (start 65.4125 59.2125) (end 67.1 60.9) (width 0.25) (layer "F.Cu") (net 1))
 (segment (start 67.1 60.9) (end 67.1 63.475) (width 0.25) (layer "F.Cu") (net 1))
 (segment (start 62.7 59.2125) (end 65.4125 59.2125) (width 0.25) (layer "F.Cu") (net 1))
 (segment (start 67.515 63.475) (end 68.45 62.54) (width 0.25) (layer "F.Cu") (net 1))
 (segment (start 67.1 63.475) (end 67.515 63.475) (width 0.25) (layer "F.Cu") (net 1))
 (segment (start 62.08 61.99) (end 57.92 61.99) (width 0.25) (layer "F.Cu") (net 2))
 (segment (start 57.6 62.31) (end 57.6 63.225) (width 0.25) (layer "F.Cu") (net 2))
 (segment (start 57.92 61.99) (end 57.6 62.31) (width 0.25) (layer "F.Cu") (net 2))
 (segment (start 62.7 60.7875) (end 62.7 61.37) (width 0.25) (layer "F.Cu") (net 2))
 (segment (start 62.7 61.37) (end 62.08 61.99) (width 0.25) (layer "F.Cu") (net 2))
 (segment (start 64.825 63.475) (end 62.555 63.475) (width 0.25) (layer "F.Cu") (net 8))
 (segment (start 59.545 63.18) (end 59.5 63.225) (width 0.25) (layer "F.Cu") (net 8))
 (segment (start 62.26 63.18) (end 59.545 63.18) (width 0.25) (layer "F.Cu") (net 8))
 (segment (start 62.555 63.475) (end 62.26 63.18) (width 0.25) (layer "F.Cu") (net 8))
 (segment (start 67.1 66.84) (end 66.965 66.975) (width 0.25) (layer "F.Cu") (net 7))
 (segment (start 67.1 65.375) (end 67.1 66.69) (width 0.25) (layer "F.Cu") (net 7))
 (segment (start 67.1 66.69) (end 67.1 66.84) (width 0.25) (layer "F.Cu") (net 7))
 (segment (start 68.82 66.69) (end 68.88 66.63) (width 0.25) (layer "F.Cu") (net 7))
 (segment (start 66.965 66.975) (end 66.475 66.975) (width 0.25) (layer "F.Cu") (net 7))
 (segment (start 67.1 66.69) (end 68.82 66.69) (width 0.25) (layer "F.Cu") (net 7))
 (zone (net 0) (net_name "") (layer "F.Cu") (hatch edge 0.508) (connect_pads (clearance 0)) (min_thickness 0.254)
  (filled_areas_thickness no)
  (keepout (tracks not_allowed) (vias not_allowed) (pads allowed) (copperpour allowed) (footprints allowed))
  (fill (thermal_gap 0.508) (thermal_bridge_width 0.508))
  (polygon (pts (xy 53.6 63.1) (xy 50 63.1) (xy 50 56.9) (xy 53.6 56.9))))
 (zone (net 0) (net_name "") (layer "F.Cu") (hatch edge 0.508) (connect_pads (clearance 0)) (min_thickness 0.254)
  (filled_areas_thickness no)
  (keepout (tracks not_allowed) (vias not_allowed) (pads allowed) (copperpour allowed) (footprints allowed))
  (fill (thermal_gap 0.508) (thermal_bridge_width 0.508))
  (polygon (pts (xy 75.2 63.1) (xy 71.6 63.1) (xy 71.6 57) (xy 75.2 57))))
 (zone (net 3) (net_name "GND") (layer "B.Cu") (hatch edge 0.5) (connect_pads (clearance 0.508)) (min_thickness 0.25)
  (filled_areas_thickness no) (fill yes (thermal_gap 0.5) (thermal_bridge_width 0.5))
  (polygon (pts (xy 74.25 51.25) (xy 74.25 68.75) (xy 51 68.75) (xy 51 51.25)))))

